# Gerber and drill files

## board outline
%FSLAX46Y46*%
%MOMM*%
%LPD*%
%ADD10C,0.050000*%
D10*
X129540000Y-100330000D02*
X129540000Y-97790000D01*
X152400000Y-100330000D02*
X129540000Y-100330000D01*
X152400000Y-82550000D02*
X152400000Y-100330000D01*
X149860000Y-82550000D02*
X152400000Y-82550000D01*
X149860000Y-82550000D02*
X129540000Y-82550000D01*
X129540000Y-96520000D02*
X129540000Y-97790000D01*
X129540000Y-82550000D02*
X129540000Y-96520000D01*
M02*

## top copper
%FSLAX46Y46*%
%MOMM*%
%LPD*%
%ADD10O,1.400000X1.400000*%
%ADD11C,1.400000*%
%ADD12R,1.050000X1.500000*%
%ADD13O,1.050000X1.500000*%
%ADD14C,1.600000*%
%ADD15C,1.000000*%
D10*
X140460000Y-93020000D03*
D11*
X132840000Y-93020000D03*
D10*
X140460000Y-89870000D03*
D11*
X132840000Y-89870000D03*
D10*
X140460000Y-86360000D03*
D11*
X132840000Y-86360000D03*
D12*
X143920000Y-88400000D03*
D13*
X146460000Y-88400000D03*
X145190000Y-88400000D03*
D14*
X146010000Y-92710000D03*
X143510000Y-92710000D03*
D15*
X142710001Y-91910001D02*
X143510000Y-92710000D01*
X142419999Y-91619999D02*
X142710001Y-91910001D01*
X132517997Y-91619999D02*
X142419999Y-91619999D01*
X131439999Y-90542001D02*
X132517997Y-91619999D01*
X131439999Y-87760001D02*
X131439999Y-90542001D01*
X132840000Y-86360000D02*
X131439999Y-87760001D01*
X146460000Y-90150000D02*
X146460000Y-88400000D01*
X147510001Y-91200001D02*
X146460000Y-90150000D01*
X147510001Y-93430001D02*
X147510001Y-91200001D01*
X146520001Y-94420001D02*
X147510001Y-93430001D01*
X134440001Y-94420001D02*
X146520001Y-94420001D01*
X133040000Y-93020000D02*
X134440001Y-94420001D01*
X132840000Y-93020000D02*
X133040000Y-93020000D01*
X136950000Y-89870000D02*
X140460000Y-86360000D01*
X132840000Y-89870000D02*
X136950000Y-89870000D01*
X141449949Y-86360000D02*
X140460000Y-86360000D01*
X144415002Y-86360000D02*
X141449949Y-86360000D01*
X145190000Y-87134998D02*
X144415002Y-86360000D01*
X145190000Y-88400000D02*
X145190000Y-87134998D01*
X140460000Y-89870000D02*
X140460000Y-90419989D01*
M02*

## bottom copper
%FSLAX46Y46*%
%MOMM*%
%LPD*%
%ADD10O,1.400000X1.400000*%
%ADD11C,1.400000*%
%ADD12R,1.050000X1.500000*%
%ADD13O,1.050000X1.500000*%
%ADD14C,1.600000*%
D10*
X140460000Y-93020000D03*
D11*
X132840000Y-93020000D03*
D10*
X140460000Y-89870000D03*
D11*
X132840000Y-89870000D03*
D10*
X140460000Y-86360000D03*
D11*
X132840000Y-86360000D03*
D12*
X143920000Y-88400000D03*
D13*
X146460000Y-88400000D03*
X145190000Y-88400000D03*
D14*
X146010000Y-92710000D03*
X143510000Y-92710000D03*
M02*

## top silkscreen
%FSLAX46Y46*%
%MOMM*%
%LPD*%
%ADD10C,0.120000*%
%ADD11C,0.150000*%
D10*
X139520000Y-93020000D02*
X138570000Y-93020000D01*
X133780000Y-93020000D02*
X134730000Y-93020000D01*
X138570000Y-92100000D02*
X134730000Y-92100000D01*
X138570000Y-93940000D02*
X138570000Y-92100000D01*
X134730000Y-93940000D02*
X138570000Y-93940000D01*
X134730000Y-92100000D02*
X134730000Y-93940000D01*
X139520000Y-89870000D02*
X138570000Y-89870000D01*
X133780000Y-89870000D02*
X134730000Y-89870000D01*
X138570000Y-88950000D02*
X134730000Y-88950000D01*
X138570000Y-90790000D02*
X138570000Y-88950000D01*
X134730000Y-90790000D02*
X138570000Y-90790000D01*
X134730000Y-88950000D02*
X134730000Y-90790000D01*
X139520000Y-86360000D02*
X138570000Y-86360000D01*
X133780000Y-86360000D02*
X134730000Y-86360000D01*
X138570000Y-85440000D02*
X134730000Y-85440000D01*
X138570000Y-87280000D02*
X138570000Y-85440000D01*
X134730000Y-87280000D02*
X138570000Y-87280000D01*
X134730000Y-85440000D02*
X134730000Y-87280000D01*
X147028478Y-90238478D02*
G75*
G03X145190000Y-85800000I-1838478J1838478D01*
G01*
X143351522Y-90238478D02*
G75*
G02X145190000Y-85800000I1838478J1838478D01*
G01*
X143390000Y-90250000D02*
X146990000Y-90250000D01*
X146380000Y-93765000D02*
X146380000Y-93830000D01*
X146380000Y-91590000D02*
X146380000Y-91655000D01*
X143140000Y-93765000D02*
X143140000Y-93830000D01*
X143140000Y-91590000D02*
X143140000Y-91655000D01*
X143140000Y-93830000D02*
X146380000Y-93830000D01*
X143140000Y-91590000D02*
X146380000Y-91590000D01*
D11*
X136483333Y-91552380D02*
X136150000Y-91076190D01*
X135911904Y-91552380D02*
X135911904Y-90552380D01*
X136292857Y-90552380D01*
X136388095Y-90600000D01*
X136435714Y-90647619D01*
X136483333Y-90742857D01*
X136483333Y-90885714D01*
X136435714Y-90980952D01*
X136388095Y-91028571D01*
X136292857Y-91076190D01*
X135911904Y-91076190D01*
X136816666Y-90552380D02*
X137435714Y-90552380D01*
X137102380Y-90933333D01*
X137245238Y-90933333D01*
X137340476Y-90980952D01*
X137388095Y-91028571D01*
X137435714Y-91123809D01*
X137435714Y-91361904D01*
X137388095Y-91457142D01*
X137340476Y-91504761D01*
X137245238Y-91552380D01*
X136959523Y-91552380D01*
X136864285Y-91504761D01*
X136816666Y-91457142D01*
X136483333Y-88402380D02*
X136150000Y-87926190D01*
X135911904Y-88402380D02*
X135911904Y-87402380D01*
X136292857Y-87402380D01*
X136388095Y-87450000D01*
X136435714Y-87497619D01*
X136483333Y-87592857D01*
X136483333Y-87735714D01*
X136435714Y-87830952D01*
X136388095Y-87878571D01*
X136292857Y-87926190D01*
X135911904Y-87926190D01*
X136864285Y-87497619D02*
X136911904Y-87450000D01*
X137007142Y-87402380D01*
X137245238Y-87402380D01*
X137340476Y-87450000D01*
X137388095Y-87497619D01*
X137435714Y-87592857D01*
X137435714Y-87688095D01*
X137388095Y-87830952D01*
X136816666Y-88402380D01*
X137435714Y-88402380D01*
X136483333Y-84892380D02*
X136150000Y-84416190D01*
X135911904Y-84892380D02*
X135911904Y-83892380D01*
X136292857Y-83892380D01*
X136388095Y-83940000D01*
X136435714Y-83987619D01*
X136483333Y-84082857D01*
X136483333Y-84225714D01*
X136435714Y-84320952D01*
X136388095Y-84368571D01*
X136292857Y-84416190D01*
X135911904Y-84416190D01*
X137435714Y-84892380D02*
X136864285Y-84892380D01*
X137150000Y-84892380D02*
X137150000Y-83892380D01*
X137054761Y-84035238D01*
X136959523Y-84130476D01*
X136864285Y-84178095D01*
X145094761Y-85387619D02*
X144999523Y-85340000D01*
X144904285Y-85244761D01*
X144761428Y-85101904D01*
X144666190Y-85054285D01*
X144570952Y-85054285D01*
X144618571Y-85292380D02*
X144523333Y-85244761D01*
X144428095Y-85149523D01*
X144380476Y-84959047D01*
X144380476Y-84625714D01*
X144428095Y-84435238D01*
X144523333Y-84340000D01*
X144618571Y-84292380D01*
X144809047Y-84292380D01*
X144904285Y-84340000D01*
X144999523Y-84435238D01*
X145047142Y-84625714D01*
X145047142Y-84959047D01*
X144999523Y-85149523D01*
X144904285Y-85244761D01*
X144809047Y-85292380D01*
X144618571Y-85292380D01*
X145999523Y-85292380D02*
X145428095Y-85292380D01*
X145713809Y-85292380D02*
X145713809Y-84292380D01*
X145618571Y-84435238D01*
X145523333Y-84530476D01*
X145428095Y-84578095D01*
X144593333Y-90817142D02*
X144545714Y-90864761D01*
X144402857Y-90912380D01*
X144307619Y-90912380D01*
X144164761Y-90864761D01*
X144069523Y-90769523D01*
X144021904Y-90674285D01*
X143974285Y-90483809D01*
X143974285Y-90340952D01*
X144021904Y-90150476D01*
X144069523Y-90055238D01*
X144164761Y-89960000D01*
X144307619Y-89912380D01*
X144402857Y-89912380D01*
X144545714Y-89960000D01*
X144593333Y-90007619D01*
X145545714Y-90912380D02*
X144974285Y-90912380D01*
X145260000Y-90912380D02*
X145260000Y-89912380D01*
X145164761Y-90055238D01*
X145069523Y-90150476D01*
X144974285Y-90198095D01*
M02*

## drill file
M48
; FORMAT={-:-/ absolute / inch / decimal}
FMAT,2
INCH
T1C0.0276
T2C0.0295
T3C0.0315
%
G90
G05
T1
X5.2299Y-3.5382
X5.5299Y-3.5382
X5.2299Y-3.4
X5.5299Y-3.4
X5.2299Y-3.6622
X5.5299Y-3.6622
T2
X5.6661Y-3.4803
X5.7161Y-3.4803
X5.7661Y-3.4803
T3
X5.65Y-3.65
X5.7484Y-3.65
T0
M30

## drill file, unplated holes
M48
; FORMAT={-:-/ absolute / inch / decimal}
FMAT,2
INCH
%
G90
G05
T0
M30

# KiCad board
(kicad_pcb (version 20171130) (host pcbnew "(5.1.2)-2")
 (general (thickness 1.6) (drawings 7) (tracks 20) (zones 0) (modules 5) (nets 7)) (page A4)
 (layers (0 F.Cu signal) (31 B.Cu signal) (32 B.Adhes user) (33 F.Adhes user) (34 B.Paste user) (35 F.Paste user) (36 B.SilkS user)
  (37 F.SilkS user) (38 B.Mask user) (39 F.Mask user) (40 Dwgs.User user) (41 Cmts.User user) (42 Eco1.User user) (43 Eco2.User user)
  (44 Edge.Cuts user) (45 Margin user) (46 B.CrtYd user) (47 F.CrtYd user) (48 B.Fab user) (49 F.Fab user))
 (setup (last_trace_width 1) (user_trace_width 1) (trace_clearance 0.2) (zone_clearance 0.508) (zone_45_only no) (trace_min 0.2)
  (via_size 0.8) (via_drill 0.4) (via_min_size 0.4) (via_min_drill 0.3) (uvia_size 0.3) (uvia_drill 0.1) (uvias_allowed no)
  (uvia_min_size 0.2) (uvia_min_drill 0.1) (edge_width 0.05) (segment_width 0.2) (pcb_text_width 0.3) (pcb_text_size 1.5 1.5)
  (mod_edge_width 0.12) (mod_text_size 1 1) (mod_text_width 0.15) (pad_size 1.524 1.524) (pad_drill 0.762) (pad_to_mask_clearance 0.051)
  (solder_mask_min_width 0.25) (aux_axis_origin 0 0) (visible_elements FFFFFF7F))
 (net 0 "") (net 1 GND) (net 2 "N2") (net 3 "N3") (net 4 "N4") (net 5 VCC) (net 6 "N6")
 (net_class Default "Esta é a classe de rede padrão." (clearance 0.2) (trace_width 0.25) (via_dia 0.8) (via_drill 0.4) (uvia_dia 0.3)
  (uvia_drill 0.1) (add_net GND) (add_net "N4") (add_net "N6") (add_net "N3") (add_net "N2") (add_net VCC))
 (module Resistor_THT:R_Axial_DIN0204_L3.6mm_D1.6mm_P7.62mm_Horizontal (layer F.Cu) (at 132.84 93.02)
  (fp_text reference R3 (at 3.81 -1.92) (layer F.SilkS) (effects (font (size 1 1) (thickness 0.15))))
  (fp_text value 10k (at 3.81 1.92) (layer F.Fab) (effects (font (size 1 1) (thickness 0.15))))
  (fp_line (start 6.68 0) (end 5.73 0) (layer F.SilkS) (width 0.12))
  (fp_line (start 0.94 0) (end 1.89 0) (layer F.SilkS) (width 0.12))
  (fp_line (start 5.73 -0.92) (end 1.89 -0.92) (layer F.SilkS) (width 0.12))
  (fp_line (start 5.73 0.92) (end 5.73 -0.92) (layer F.SilkS) (width 0.12))
  (fp_line (start 1.89 0.92) (end 5.73 0.92) (layer F.SilkS) (width 0.12))
  (fp_line (start 1.89 -0.92) (end 1.89 0.92) (layer F.SilkS) (width 0.12))
  (pad 2 thru_hole oval (at 7.62 0) (size 1.4 1.4) (drill 0.7) (layers *.Cu *.Mask) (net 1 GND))
  (pad 1 thru_hole circle (at 0 0) (size 1.4 1.4) (drill 0.7) (layers *.Cu *.Mask) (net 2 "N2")))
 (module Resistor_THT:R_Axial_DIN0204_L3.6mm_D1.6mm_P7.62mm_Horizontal (layer F.Cu) (at 132.84 89.87)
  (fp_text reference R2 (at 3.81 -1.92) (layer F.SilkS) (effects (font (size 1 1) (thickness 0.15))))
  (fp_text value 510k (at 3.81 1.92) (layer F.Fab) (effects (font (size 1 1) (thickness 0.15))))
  (fp_line (start 6.68 0) (end 5.73 0) (layer F.SilkS) (width 0.12))
  (fp_line (start 0.94 0) (end 1.89 0) (layer F.SilkS) (width 0.12))
  (fp_line (start 5.73 -0.92) (end 1.89 -0.92) (layer F.SilkS) (width 0.12))
  (fp_line (start 5.73 0.92) (end 5.73 -0.92) (layer F.SilkS) (width 0.12))
  (fp_line (start 1.89 0.92) (end 5.73 0.92) (layer F.SilkS) (width 0.12))
  (fp_line (start 1.89 -0.92) (end 1.89 0.92) (layer F.SilkS) (width 0.12))
  (pad 2 thru_hole oval (at 7.62 0) (size 1.4 1.4) (drill 0.7) (layers *.Cu *.Mask) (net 1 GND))
  (pad 1 thru_hole circle (at 0 0) (size 1.4 1.4) (drill 0.7) (layers *.Cu *.Mask) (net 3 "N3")))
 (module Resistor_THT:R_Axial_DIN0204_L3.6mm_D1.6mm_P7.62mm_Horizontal (layer F.Cu) (at 132.84 86.36)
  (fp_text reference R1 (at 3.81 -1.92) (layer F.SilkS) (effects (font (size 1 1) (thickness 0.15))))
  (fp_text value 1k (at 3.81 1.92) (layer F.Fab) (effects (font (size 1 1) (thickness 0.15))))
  (fp_line (start 6.68 0) (end 5.73 0) (layer F.SilkS) (width 0.12))
  (fp_line (start 0.94 0) (end 1.89 0) (layer F.SilkS) (width 0.12))
  (fp_line (start 5.73 -0.92) (end 1.89 -0.92) (layer F.SilkS) (width 0.12))
  (fp_line (start 5.73 0.92) (end 5.73 -0.92) (layer F.SilkS) (width 0.12))
  (fp_line (start 1.89 0.92) (end 5.73 0.92) (layer F.SilkS) (width 0.12))
  (fp_line (start 1.89 -0.92) (end 1.89 0.92) (layer F.SilkS) (width 0.12))
  (pad 2 thru_hole oval (at 7.62 0) (size 1.4 1.4) (drill 0.7) (layers *.Cu *.Mask) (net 3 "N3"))
  (pad 1 thru_hole circle (at 0 0) (size 1.4 1.4) (drill 0.7) (layers *.Cu *.Mask) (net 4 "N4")))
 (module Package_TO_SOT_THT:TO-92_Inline (layer F.Cu) (at 143.92 88.4)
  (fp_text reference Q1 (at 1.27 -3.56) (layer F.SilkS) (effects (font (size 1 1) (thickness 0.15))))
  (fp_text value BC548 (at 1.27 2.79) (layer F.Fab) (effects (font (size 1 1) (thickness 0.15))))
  (fp_arc (start 1.27 0) (end 1.27 -2.6) (angle 135) (layer F.SilkS) (width 0.12))
  (fp_arc (start 1.27 0) (end 1.27 -2.6) (angle -135) (layer F.SilkS) (width 0.12))
  (fp_line (start -0.53 1.85) (end 3.07 1.85) (layer F.SilkS) (width 0.12))
  (pad 1 thru_hole rect (at 0 0) (size 1.05 1.5) (drill 0.75) (layers *.Cu *.Mask) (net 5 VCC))
  (pad 3 thru_hole oval (at 2.54 0) (size 1.05 1.5) (drill 0.75) (layers *.Cu *.Mask) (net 2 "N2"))
  (pad 2 thru_hole oval (at 1.27 0) (size 1.05 1.5) (drill 0.75) (layers *.Cu *.Mask) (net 3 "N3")))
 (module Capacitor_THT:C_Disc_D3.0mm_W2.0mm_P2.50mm (layer F.Cu) (at 143.51 92.71)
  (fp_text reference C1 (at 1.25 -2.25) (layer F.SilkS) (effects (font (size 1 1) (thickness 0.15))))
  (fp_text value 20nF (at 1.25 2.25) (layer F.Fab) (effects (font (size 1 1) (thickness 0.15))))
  (fp_line (start 2.87 1.055) (end 2.87 1.12) (layer F.SilkS) (width 0.12))
  (fp_line (start 2.87 -1.12) (end 2.87 -1.055) (layer F.SilkS) (width 0.12))
  (fp_line (start -0.37 1.055) (end -0.37 1.12) (layer F.SilkS) (width 0.12))
  (fp_line (start -0.37 -1.12) (end -0.37 -1.055) (layer F.SilkS) (width 0.12))
  (fp_line (start -0.37 1.12) (end 2.87 1.12) (layer F.SilkS) (width 0.12))
  (fp_line (start -0.37 -1.12) (end 2.87 -1.12) (layer F.SilkS) (width 0.12))
  (pad 2 thru_hole circle (at 2.5 0) (size 1.6 1.6) (drill 0.8) (layers *.Cu *.Mask) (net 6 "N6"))
  (pad 1 thru_hole circle (at 0 0) (size 1.6 1.6) (drill 0.8) (layers *.Cu *.Mask) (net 4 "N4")))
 (gr_line (start 129.54 100.33) (end 129.54 97.79) (layer Edge.Cuts) (width 0.05))
 (gr_line (start 152.4 100.33) (end 129.54 100.33) (layer Edge.Cuts) (width 0.05))
 (gr_line (start 152.4 82.55) (end 152.4 100.33) (layer Edge.Cuts) (width 0.05))
 (gr_line (start 149.86 82.55) (end 152.4 82.55) (layer Edge.Cuts) (width 0.05))
 (gr_line (start 149.86 82.55) (end 129.54 82.55) (layer Edge.Cuts) (width 0.05))
 (gr_line (start 129.54 96.52) (end 129.54 97.79) (layer Edge.Cuts) (width 0.05))
 (gr_line (start 129.54 82.55) (end 129.54 96.52) (layer Edge.Cuts) (width 0.05))
 (segment (start 142.710001 91.910001) (end 143.51 92.71) (width 1) (layer F.Cu) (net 4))
 (segment (start 142.419999 91.619999) (end 142.710001 91.910001) (width 1) (layer F.Cu) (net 4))
 (segment (start 132.517997 91.619999) (end 142.419999 91.619999) (width 1) (layer F.Cu) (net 4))
 (segment (start 131.439999 90.542001) (end 132.517997 91.619999) (width 1) (layer F.Cu) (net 4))
 (segment (start 131.439999 87.760001) (end 131.439999 90.542001) (width 1) (layer F.Cu) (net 4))
 (segment (start 132.84 86.36) (end 131.439999 87.760001) (width 1) (layer F.Cu) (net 4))
 (segment (start 146.46 90.15) (end 146.46 88.4) (width 1) (layer F.Cu) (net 2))
 (segment (start 147.510001 91.200001) (end 146.46 90.15) (width 1) (layer F.Cu) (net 2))
 (segment (start 147.510001 93.430001) (end 147.510001 91.200001) (width 1) (layer F.Cu) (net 2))
 (segment (start 146.520001 94.420001) (end 147.510001 93.430001) (width 1) (layer F.Cu) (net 2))
 (segment (start 134.440001 94.420001) (end 146.520001 94.420001) (width 1) (layer F.Cu) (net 2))
 (segment (start 133.04 93.02) (end 134.440001 94.420001) (width 1) (layer F.Cu) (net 2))
 (segment (start 132.84 93.02) (end 133.04 93.02) (width 1) (layer F.Cu) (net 2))
 (segment (start 136.95 89.87) (end 140.46 86.36) (width 1) (layer F.Cu) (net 3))
 (segment (start 132.84 89.87) (end 136.95 89.87) (width 1) (layer F.Cu) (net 3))
 (segment (start 141.449949 86.36) (end 140.46 86.36) (width 1) (layer F.Cu) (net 3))
 (segment (start 144.415002 86.36) (end 141.449949 86.36) (width 1) (layer F.Cu) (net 3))
 (segment (start 145.19 87.134998) (end 144.415002 86.36) (width 1) (layer F.Cu) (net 3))
 (segment (start 145.19 88.4) (end 145.19 87.134998) (width 1) (layer F.Cu) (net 3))
 (segment (start 140.46 89.87) (end 140.46 90.419989) (width 1) (layer F.Cu) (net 1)))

